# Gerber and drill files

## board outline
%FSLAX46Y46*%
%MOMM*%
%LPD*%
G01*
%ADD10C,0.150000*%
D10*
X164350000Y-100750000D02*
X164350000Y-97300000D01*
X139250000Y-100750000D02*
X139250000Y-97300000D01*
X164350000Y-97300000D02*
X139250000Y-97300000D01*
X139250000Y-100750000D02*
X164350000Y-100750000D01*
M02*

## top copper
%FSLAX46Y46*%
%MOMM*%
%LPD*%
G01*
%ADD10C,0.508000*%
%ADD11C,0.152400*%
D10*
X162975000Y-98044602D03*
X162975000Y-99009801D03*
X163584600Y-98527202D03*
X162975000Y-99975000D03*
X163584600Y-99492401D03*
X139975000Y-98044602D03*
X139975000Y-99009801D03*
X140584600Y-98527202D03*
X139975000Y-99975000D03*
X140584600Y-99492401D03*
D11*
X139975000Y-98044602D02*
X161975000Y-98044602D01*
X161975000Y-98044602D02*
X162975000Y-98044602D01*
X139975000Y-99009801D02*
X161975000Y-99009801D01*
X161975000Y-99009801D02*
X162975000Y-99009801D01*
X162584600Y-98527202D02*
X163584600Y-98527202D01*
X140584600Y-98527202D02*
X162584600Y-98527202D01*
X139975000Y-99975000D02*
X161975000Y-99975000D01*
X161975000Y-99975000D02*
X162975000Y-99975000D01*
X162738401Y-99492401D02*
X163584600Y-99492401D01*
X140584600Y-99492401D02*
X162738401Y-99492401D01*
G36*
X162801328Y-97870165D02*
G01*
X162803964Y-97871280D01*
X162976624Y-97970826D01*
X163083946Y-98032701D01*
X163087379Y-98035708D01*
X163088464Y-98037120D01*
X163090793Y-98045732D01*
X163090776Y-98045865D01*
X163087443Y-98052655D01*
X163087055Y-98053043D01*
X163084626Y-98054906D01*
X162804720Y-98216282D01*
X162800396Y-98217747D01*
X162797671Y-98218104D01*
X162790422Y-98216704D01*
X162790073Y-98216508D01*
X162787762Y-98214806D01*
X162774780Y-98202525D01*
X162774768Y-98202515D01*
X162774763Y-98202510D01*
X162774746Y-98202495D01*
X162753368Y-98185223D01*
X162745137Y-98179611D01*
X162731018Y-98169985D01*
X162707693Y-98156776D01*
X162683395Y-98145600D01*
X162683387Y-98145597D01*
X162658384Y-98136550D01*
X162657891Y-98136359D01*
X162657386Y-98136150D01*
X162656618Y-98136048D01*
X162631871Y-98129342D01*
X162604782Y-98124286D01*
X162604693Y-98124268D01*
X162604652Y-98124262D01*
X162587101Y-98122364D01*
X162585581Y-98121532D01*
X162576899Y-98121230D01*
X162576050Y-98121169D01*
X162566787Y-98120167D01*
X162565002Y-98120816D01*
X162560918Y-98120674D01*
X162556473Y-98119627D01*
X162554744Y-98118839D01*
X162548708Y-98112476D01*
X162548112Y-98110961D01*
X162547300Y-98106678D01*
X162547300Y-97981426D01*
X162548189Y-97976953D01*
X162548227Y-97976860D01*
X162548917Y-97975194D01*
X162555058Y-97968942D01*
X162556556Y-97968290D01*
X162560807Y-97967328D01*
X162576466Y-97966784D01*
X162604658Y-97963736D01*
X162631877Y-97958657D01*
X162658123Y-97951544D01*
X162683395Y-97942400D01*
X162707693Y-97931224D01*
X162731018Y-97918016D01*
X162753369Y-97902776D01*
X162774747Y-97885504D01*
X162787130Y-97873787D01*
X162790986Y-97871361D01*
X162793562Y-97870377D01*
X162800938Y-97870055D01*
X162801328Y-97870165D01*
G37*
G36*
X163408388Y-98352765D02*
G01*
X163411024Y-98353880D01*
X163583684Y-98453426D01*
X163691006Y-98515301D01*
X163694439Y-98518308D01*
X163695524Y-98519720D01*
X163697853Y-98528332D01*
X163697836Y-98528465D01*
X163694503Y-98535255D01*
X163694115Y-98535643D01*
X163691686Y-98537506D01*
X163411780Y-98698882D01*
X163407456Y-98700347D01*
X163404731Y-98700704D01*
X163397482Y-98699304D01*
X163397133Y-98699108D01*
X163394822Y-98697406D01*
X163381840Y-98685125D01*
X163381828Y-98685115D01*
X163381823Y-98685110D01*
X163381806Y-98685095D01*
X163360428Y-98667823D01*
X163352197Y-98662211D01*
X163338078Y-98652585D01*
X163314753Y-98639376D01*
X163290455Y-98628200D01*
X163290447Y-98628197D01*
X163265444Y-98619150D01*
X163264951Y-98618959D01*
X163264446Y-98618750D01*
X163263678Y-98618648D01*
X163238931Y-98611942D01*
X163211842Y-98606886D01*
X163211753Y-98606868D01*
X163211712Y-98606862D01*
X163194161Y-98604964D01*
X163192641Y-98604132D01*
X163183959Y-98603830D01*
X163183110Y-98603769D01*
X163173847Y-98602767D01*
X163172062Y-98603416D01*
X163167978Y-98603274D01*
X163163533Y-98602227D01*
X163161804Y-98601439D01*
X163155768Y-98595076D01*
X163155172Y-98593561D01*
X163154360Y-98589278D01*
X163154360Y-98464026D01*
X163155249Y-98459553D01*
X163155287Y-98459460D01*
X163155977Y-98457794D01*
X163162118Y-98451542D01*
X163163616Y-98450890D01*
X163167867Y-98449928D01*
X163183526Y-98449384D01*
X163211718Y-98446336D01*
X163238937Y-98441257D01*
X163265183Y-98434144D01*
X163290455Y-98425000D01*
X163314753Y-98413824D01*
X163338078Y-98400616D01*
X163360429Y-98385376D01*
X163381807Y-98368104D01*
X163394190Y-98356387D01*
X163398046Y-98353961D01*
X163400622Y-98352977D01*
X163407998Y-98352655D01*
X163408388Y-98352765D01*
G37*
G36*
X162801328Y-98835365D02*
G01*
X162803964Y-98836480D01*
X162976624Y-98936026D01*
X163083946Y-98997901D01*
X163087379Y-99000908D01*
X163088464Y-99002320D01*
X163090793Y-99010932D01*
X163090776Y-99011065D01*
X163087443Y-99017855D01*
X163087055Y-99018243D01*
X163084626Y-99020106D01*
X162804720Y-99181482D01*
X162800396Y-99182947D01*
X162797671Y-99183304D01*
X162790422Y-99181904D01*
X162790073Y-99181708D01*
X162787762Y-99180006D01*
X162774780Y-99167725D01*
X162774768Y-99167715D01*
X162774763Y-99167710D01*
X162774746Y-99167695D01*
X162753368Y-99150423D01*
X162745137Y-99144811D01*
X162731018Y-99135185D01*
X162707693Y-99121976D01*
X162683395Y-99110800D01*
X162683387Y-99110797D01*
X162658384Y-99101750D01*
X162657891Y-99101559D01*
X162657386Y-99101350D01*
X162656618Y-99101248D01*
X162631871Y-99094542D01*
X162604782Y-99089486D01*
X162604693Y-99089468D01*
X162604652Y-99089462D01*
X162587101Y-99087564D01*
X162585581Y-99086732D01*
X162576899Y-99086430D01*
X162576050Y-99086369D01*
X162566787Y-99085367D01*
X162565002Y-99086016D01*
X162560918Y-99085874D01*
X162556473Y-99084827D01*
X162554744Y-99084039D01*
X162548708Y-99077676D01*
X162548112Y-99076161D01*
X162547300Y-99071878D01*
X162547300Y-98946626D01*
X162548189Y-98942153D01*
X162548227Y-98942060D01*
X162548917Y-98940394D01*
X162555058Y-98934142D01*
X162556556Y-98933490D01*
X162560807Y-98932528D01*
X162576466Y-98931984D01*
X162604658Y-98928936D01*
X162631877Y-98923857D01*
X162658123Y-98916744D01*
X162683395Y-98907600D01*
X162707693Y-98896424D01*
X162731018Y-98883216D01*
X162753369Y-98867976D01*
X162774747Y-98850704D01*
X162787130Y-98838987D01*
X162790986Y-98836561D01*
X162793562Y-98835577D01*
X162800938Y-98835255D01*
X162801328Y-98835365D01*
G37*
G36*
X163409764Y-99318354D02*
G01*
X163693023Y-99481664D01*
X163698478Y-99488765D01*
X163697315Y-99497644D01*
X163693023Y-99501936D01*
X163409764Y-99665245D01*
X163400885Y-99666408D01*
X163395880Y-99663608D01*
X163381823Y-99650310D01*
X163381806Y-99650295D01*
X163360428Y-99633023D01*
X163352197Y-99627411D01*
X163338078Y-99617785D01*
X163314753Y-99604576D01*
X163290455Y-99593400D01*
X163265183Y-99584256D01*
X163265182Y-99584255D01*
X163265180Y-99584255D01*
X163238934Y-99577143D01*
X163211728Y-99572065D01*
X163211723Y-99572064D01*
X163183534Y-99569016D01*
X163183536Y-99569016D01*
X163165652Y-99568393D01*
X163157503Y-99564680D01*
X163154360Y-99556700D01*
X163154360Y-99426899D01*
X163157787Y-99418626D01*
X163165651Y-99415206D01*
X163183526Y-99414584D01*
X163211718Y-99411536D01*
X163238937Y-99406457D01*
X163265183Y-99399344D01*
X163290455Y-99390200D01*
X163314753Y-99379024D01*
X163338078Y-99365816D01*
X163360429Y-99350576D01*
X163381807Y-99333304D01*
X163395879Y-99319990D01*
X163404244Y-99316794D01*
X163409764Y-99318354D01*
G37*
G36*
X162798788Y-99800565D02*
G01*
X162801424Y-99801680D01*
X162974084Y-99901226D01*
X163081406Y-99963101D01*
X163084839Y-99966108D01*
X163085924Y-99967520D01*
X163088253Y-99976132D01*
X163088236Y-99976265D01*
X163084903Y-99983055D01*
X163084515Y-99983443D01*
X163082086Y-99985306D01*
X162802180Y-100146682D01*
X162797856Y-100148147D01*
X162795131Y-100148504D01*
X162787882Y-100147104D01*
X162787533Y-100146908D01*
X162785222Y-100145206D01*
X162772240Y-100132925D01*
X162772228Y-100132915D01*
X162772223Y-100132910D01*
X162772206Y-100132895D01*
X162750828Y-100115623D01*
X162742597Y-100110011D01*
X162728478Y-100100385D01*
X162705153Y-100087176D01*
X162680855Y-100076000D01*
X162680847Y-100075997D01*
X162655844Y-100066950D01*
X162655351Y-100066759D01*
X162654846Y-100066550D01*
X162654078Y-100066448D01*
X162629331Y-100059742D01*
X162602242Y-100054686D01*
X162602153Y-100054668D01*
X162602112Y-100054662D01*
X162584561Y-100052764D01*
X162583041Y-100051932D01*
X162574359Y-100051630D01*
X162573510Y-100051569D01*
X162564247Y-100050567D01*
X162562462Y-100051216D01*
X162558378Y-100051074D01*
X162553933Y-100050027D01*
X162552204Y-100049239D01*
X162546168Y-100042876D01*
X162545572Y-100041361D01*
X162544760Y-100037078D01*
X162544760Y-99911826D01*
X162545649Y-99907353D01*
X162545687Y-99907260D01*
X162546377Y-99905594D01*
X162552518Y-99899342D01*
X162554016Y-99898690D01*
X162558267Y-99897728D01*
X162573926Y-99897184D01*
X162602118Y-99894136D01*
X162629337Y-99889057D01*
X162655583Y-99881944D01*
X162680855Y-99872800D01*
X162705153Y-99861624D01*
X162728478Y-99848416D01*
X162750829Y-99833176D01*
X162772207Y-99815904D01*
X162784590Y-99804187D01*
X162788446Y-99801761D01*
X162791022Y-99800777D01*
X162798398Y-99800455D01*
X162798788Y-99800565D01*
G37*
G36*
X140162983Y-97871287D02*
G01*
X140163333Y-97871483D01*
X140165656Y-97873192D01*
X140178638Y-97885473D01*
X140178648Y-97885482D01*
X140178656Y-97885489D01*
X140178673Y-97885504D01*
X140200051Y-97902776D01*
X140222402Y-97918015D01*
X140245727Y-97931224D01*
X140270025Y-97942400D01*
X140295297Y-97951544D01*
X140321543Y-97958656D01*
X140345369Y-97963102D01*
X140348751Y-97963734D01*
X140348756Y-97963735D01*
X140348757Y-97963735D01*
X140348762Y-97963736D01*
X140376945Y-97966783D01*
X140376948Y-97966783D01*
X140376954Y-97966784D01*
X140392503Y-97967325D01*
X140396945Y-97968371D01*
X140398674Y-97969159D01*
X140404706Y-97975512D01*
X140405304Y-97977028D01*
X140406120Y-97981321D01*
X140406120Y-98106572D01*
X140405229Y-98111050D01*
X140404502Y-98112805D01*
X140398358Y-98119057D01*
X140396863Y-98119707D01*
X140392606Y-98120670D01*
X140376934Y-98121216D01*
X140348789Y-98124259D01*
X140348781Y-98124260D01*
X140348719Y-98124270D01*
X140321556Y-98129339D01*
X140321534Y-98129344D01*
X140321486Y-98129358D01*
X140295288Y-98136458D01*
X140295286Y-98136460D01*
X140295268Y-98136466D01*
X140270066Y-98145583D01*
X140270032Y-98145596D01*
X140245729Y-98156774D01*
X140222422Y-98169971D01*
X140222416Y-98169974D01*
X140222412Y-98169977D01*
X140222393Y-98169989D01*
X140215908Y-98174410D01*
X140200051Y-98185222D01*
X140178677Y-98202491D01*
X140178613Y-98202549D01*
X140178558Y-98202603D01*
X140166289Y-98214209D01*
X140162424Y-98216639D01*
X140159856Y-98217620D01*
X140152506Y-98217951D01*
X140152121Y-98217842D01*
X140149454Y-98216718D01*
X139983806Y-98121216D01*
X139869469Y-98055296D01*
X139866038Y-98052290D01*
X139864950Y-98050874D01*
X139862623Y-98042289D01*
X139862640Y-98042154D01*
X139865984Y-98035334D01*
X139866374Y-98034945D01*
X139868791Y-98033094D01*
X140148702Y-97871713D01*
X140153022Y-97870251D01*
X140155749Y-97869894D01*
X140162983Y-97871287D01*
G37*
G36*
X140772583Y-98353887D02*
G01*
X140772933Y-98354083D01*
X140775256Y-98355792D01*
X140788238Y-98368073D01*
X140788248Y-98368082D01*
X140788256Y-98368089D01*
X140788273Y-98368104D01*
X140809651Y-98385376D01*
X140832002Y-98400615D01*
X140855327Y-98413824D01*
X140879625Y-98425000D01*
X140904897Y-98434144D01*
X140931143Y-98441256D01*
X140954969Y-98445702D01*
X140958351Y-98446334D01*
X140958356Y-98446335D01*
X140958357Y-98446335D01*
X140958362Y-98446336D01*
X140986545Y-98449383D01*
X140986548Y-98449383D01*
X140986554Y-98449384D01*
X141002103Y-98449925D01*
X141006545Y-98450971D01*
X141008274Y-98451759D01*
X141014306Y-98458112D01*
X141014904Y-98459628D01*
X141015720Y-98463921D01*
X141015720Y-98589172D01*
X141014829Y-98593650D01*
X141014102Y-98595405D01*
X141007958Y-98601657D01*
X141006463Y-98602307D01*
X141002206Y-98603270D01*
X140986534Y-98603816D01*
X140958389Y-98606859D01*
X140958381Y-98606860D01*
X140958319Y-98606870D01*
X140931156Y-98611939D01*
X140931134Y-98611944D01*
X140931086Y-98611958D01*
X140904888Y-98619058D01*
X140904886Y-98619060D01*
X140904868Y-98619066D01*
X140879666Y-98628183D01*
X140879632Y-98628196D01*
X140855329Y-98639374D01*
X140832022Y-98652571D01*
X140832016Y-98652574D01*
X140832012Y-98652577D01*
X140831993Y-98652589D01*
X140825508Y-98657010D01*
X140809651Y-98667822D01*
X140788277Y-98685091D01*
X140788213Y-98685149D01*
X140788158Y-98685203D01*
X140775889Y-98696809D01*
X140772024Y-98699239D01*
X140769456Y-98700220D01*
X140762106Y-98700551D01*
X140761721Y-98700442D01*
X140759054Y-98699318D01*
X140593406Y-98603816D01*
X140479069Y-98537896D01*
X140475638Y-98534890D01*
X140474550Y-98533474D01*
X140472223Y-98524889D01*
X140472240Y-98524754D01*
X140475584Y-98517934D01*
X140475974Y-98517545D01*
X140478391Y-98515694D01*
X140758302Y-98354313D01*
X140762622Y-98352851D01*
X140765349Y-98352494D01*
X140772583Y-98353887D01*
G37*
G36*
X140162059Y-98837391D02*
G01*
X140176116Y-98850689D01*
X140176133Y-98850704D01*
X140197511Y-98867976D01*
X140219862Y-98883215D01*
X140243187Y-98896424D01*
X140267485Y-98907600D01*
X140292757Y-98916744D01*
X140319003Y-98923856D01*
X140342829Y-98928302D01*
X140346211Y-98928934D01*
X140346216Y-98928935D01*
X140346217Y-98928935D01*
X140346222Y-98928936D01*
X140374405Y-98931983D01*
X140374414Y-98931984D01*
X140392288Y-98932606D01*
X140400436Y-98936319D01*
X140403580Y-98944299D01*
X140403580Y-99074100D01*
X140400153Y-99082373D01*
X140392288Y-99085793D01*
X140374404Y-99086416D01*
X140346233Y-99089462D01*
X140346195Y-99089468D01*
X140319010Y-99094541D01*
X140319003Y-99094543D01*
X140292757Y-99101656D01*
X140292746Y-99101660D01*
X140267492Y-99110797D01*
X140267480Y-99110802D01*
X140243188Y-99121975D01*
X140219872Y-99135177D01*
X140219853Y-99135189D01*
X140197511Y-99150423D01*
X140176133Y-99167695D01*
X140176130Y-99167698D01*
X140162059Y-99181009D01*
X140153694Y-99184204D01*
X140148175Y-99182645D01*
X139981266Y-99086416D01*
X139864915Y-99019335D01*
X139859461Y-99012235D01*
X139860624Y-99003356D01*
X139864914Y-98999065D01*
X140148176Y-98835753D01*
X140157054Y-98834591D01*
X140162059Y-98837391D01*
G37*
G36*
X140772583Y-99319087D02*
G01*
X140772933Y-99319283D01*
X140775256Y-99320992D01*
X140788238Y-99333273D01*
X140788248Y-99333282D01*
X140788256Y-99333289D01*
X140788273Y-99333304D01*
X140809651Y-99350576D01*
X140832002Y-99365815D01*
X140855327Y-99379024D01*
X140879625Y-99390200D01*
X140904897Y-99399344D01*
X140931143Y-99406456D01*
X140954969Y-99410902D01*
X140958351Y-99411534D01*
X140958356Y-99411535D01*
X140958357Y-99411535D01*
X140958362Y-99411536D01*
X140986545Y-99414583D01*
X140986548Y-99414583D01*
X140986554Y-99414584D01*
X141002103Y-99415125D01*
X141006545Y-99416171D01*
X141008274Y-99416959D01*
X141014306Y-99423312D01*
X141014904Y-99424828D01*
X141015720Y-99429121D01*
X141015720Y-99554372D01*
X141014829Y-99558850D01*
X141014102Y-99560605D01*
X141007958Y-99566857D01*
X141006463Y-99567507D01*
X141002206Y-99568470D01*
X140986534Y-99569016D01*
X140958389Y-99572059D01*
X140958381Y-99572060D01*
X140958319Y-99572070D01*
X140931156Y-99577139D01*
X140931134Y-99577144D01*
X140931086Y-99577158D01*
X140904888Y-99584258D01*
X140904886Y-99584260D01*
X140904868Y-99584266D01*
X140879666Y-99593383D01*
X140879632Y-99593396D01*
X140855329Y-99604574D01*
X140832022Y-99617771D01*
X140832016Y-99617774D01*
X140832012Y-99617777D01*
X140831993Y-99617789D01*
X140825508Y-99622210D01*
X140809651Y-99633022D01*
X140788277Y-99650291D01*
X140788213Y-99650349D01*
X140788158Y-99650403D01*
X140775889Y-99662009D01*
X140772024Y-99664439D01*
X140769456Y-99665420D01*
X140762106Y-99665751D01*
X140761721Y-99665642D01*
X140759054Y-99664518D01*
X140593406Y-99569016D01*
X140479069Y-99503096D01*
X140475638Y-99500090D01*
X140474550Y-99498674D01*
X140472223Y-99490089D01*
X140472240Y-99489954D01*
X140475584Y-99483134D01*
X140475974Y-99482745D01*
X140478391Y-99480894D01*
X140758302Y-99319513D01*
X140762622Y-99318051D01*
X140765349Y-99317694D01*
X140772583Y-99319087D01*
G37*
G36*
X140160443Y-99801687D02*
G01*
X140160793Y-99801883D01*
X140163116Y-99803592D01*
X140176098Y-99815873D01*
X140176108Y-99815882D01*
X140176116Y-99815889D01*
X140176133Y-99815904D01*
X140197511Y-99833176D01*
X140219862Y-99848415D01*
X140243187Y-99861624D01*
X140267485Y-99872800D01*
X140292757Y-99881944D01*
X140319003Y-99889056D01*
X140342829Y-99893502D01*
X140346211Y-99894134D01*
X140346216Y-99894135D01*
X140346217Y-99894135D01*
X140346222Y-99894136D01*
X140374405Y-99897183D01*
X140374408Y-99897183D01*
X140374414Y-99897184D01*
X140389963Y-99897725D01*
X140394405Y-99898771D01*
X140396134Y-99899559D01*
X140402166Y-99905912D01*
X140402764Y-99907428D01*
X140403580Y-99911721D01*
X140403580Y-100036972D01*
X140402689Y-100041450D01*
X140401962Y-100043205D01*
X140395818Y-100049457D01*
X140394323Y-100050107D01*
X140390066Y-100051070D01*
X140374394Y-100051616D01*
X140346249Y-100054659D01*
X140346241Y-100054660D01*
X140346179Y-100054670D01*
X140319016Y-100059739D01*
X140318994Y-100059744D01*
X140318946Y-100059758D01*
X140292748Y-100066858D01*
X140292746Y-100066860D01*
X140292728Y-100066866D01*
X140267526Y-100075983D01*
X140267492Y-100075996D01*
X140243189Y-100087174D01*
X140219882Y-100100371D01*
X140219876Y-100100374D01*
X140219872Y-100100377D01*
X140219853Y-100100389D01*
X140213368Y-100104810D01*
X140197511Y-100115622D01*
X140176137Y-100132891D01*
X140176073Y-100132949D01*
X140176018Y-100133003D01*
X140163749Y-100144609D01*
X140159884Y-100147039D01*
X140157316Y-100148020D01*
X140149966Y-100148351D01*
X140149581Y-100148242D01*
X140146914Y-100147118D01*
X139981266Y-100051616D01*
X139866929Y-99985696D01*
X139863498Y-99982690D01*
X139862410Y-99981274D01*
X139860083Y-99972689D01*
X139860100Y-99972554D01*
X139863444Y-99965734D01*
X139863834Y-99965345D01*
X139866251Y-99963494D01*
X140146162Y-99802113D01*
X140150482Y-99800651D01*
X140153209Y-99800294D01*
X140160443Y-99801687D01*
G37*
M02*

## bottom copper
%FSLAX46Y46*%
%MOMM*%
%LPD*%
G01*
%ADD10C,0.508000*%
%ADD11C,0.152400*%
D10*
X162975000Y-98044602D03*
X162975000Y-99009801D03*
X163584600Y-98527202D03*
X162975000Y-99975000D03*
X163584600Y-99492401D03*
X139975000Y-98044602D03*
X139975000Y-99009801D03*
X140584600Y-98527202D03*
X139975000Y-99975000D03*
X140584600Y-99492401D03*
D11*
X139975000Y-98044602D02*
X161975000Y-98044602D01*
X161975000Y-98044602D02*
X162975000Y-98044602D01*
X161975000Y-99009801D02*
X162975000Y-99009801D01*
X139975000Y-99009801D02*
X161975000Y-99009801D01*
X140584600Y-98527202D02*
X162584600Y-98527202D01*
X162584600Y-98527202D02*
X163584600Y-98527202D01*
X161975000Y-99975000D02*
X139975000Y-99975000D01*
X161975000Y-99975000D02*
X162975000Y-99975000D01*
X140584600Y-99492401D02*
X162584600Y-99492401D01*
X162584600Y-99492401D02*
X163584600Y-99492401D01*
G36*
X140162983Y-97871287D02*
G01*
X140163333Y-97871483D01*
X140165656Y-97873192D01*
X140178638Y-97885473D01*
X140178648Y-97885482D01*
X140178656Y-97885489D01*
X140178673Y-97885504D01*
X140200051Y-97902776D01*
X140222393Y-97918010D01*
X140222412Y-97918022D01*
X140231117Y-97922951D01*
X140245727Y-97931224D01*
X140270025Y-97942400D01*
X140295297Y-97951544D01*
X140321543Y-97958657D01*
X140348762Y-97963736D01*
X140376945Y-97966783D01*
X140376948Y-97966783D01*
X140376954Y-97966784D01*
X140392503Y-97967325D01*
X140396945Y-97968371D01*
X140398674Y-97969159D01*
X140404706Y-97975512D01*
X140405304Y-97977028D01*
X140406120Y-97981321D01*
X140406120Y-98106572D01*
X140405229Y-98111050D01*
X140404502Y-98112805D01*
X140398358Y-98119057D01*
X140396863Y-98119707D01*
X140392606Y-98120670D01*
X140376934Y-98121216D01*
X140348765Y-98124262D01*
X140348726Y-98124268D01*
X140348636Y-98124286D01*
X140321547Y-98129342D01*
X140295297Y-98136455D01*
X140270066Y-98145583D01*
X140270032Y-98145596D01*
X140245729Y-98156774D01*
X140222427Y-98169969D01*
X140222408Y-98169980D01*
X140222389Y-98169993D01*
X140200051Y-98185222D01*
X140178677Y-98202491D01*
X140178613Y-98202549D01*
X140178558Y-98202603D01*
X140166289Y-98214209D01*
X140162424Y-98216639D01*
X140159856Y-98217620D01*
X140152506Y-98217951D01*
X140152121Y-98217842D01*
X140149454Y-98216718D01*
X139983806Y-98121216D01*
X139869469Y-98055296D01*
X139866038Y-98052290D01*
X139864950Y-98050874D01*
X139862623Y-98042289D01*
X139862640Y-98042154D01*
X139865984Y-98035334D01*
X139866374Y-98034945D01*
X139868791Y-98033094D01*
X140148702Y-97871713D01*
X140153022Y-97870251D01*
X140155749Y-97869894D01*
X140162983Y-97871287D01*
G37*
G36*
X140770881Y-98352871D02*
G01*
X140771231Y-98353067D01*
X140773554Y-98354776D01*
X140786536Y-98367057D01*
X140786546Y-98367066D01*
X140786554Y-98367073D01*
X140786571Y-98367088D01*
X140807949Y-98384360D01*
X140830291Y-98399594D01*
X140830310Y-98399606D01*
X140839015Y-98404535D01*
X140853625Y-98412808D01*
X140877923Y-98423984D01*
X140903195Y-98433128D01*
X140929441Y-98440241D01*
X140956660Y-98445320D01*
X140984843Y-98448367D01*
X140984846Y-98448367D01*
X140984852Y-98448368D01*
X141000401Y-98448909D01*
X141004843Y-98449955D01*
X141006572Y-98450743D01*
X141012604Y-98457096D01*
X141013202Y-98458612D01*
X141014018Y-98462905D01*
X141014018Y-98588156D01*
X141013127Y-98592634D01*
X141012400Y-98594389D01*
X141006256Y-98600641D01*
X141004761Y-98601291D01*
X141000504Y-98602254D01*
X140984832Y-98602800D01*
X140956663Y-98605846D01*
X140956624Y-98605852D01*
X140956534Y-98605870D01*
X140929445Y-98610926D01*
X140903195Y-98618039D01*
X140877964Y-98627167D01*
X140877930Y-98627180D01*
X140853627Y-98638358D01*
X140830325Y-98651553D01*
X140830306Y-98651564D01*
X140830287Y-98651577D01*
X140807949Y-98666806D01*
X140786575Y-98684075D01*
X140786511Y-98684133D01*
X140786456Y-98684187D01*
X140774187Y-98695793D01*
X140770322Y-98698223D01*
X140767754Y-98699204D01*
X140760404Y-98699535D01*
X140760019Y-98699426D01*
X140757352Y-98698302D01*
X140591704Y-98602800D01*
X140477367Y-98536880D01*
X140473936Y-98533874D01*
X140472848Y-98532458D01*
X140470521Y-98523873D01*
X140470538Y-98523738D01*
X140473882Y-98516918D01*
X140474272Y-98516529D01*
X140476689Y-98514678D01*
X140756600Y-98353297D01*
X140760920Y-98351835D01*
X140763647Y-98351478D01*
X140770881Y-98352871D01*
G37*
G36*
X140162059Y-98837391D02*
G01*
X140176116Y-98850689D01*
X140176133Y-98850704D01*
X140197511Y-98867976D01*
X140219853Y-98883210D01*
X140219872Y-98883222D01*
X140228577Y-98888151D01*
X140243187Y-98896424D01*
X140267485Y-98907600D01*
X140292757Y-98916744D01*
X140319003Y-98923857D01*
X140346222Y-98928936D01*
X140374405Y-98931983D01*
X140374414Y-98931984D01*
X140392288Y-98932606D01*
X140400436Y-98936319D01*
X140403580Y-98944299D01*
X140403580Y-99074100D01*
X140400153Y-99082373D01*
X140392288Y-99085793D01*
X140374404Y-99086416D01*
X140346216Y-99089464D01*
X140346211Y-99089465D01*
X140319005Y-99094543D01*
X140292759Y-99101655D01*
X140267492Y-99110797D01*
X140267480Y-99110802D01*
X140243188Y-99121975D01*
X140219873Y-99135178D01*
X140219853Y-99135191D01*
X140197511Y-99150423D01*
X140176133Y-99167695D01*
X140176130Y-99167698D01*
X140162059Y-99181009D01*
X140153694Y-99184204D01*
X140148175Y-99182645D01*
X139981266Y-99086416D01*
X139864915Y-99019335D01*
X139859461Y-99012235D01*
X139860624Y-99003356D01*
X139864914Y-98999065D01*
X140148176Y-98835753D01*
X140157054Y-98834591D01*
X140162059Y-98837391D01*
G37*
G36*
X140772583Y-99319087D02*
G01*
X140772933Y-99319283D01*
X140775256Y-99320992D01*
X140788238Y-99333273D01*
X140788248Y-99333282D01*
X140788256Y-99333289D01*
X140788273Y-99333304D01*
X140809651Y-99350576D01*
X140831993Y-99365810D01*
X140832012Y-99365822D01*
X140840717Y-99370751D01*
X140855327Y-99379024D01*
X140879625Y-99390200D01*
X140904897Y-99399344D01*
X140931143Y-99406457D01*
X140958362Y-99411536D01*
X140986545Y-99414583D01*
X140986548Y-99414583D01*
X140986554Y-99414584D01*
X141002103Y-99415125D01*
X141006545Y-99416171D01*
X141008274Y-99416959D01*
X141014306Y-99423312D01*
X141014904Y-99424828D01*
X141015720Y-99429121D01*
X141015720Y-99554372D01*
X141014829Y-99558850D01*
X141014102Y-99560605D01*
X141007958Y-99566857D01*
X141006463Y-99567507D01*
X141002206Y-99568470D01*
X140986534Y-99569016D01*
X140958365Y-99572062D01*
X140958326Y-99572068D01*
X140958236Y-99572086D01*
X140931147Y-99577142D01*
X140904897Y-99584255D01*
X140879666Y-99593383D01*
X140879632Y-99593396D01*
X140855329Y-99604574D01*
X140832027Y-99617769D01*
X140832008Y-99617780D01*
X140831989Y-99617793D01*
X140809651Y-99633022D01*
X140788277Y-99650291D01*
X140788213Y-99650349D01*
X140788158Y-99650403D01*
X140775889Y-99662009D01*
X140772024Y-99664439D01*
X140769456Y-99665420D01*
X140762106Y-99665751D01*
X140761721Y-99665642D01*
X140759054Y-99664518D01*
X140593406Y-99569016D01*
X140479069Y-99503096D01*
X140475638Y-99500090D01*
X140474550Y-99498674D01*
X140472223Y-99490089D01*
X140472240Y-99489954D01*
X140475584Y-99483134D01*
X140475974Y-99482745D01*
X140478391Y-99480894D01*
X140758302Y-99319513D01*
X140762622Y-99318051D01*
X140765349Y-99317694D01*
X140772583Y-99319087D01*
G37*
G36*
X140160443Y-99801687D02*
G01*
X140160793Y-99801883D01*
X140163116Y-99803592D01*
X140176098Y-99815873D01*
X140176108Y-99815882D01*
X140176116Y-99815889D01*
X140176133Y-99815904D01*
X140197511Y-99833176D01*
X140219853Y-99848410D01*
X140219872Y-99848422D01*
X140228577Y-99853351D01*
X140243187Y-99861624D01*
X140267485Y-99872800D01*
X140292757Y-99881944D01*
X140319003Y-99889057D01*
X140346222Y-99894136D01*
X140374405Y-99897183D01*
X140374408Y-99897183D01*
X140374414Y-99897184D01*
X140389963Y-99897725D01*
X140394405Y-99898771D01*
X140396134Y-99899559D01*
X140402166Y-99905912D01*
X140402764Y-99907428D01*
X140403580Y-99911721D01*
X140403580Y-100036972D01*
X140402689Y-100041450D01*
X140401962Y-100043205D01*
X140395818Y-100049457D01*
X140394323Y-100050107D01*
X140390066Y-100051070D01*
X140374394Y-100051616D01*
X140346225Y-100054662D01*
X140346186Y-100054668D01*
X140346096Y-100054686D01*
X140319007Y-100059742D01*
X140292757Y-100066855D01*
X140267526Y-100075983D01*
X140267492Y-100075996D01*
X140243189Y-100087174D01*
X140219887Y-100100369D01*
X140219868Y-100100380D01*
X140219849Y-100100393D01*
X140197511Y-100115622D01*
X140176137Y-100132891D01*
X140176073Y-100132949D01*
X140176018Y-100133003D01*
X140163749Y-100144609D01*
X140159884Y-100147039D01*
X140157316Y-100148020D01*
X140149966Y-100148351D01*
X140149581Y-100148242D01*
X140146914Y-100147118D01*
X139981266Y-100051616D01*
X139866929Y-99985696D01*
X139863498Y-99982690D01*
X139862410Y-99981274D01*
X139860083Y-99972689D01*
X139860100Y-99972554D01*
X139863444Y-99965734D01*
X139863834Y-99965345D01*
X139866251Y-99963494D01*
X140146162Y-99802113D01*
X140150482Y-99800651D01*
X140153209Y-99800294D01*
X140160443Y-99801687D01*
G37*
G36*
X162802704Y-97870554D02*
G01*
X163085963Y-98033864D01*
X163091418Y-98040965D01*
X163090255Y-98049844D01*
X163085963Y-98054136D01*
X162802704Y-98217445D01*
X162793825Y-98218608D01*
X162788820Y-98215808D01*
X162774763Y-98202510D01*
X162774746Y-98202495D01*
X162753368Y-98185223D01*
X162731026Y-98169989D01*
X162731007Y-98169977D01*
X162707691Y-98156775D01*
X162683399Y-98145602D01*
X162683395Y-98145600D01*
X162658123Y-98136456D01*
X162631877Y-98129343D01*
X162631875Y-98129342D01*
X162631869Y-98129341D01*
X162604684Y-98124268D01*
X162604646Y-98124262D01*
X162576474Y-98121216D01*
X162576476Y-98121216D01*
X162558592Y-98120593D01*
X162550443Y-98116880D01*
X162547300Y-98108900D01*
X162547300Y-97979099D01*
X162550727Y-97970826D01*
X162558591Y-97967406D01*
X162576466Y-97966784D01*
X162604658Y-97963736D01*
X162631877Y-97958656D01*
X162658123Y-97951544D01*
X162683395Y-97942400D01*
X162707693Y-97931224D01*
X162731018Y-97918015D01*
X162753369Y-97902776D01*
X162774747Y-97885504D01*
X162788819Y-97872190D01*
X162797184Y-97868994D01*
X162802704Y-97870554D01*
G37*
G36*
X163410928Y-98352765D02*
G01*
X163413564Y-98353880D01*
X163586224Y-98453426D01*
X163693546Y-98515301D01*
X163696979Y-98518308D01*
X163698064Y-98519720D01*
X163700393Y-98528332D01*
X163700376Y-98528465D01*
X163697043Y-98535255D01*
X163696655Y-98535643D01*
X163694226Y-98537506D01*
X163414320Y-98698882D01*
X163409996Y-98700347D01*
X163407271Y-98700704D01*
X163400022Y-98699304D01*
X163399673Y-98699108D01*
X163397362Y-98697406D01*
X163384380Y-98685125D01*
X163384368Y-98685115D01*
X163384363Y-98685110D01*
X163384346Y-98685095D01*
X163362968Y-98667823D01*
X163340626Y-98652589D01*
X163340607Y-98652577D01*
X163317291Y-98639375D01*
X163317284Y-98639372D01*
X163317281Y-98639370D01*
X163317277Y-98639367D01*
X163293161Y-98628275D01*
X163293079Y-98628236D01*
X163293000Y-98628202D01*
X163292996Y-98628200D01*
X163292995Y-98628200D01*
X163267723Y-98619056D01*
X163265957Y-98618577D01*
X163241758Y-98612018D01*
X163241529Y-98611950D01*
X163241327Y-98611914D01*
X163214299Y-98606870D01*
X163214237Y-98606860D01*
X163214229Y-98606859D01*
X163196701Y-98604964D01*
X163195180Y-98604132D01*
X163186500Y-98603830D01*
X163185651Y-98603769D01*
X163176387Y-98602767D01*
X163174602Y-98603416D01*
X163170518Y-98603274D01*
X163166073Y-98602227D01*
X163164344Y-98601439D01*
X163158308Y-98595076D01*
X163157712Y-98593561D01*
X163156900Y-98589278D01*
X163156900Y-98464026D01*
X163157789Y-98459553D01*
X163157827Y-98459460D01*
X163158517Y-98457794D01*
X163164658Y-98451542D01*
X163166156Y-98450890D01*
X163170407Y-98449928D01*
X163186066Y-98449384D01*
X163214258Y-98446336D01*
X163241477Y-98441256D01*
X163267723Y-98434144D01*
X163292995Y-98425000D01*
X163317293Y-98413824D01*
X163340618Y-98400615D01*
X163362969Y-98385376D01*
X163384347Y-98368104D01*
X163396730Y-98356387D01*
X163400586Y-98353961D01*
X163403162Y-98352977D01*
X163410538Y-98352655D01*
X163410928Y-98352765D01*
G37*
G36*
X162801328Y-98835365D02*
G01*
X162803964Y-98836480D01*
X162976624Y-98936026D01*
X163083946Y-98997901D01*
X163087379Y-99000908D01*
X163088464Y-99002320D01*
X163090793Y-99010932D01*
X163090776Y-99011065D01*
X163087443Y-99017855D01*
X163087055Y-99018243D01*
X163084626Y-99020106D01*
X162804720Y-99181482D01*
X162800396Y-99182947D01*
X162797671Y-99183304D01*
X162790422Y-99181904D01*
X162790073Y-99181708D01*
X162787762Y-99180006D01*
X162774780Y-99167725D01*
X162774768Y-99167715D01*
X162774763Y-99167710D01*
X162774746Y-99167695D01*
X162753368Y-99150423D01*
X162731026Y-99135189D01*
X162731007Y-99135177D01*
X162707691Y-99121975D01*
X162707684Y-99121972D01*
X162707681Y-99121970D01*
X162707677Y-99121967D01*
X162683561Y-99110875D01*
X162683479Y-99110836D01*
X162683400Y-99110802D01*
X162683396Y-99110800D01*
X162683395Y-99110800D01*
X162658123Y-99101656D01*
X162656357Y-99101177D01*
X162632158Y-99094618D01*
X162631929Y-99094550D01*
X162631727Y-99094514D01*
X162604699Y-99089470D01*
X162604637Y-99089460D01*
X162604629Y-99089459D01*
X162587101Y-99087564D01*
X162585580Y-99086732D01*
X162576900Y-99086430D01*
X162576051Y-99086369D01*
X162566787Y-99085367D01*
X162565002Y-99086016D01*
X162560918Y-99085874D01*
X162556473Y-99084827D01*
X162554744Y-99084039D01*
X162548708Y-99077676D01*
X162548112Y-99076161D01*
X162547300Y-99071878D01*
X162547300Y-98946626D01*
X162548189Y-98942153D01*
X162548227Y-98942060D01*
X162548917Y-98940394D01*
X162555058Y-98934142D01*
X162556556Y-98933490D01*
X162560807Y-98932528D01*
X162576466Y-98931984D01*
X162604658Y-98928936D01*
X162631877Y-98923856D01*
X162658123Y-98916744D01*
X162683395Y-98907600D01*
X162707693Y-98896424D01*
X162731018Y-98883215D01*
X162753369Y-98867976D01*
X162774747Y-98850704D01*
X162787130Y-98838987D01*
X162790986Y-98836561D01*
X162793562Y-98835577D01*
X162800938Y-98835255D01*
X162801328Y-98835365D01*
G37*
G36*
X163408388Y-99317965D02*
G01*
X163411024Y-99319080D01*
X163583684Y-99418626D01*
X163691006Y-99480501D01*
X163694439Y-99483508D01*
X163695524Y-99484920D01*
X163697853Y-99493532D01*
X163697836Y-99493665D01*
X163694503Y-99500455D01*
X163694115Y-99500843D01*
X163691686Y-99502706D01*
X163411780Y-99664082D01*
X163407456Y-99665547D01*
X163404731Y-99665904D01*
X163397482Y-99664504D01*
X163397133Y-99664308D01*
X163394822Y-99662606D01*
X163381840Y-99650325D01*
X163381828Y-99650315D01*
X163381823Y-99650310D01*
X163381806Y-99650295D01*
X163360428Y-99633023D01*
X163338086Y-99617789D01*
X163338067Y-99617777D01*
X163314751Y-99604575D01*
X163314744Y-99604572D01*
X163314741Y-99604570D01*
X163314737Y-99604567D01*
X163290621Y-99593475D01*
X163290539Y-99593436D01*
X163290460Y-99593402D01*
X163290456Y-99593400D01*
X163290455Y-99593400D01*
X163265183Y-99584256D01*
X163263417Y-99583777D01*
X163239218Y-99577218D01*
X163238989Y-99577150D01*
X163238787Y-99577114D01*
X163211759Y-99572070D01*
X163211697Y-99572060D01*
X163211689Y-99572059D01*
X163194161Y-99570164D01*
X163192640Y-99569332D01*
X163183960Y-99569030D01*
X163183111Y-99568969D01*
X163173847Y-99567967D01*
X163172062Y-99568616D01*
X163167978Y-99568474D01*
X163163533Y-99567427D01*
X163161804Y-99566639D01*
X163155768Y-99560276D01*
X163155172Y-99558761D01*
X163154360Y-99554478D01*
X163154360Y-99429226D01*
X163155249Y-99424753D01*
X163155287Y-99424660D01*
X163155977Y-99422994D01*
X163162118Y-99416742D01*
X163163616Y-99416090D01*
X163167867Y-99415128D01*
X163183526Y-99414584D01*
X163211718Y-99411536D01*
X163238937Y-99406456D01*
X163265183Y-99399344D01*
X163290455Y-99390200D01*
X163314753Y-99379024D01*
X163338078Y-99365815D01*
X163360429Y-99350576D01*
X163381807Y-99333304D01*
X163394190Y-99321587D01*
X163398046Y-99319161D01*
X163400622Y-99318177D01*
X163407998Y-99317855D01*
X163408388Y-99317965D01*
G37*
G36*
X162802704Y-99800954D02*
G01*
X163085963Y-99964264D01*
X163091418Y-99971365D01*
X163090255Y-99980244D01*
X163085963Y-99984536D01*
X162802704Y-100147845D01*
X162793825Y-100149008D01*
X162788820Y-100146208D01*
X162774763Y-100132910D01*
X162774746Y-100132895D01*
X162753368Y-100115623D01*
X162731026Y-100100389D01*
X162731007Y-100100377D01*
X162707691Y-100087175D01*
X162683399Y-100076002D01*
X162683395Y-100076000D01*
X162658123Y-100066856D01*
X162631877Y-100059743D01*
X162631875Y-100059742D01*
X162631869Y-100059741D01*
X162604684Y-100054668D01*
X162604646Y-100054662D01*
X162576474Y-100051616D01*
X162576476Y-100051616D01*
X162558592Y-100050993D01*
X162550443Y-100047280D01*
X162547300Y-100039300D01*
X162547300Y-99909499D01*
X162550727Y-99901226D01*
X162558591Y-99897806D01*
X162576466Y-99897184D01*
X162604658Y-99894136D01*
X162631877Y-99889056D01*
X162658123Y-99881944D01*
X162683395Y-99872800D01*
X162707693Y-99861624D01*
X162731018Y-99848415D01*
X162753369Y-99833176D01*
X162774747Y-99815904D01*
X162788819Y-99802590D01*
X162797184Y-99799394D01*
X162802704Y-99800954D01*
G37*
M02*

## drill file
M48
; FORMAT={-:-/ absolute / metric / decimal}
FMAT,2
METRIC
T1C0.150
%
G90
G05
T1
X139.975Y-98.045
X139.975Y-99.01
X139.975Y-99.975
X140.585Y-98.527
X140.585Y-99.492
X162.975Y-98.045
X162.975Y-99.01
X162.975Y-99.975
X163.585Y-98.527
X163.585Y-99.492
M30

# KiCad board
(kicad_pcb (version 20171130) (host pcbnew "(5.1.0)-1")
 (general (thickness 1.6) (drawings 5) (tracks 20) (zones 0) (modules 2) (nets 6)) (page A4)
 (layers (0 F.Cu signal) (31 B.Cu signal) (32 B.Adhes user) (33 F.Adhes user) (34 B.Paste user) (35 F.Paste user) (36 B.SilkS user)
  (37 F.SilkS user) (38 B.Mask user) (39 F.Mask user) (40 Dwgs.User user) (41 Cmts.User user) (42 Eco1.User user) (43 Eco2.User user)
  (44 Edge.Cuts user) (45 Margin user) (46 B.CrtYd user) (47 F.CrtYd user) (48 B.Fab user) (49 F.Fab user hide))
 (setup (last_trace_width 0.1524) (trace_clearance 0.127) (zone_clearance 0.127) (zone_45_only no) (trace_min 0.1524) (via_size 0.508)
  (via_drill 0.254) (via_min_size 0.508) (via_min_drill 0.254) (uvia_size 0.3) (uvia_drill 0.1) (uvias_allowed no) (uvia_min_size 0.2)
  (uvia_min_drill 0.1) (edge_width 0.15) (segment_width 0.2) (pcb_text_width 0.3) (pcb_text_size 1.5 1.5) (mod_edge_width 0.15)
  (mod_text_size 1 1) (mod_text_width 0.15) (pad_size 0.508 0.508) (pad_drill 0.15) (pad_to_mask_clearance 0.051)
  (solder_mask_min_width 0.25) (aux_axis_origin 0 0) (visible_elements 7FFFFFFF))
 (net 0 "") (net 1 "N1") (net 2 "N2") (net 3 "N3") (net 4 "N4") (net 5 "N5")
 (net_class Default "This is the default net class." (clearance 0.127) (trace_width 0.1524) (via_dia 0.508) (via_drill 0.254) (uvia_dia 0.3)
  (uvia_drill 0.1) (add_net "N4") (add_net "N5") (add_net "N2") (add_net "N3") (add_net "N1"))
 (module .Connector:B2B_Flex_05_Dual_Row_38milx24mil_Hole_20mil (layer F.Cu) (at 163 100 90)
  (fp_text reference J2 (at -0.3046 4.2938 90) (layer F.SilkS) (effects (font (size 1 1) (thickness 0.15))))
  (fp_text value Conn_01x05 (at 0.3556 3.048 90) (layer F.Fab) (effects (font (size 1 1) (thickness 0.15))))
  (pad 5 thru_hole circle (at 1.955398 -0.025 90) (size 0.508 0.508) (drill 0.15) (layers *.Cu *.Mask) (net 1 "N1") (zone_connect 2))
  (pad 3 thru_hole circle (at 0.990199 -0.025 90) (size 0.508 0.508) (drill 0.15) (layers *.Cu *.Mask) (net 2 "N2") (zone_connect 2))
  (pad 4 thru_hole circle (at 1.472798 0.5846 90) (size 0.508 0.508) (drill 0.15) (layers *.Cu *.Mask) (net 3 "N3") (zone_connect 2))
  (pad 1 thru_hole circle (at 0.025 -0.025 90) (size 0.508 0.508) (drill 0.15) (layers *.Cu *.Mask) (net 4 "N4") (zone_connect 2))
  (pad 2 thru_hole circle (at 0.507599 0.5846 90) (size 0.508 0.508) (drill 0.15) (layers *.Cu *.Mask) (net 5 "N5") (zone_connect 2)))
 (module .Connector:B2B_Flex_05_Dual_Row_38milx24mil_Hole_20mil (layer F.Cu) (at 140 100 90)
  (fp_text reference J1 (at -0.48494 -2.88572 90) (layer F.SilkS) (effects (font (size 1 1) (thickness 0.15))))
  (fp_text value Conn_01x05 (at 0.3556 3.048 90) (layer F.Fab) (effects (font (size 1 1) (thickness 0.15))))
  (pad 5 thru_hole circle (at 1.955398 -0.025 90) (size 0.508 0.508) (drill 0.15) (layers *.Cu *.Mask) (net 1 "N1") (zone_connect 2))
  (pad 3 thru_hole circle (at 0.990199 -0.025 90) (size 0.508 0.508) (drill 0.15) (layers *.Cu *.Mask) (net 2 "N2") (zone_connect 2))
  (pad 4 thru_hole circle (at 1.472798 0.5846 90) (size 0.508 0.508) (drill 0.15) (layers *.Cu *.Mask) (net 3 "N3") (zone_connect 2))
  (pad 1 thru_hole circle (at 0.025 -0.025 90) (size 0.508 0.508) (drill 0.15) (layers *.Cu *.Mask) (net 4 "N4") (zone_connect 2))
  (pad 2 thru_hole circle (at 0.507599 0.5846 90) (size 0.508 0.508) (drill 0.15) (layers *.Cu *.Mask) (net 5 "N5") (zone_connect 2)))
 (gr_line (start 164.35 100.75) (end 164.35 97.3) (layer Edge.Cuts) (width 0.15))
 (gr_line (start 139.25 100.75) (end 139.25 97.3) (layer Edge.Cuts) (width 0.15))
 (gr_line (start 164.35 97.3) (end 139.25 97.3) (layer Edge.Cuts) (width 0.15))
 (gr_line (start 139.25 100.75) (end 164.35 100.75) (layer Edge.Cuts) (width 0.15))
 (segment (start 139.975 98.044602) (end 161.975 98.044602) (width 0.1524) (layer F.Cu) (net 1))
 (segment (start 139.975 98.044602) (end 161.975 98.044602) (width 0.1524) (layer B.Cu) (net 1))
 (segment (start 161.975 98.044602) (end 162.975 98.044602) (width 0.1524) (layer B.Cu) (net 1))
 (segment (start 161.975 98.044602) (end 162.975 98.044602) (width 0.1524) (layer F.Cu) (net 1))
 (segment (start 139.975 99.009801) (end 161.975 99.009801) (width 0.1524) (layer F.Cu) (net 2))
 (segment (start 161.975 99.009801) (end 162.975 99.009801) (width 0.1524) (layer B.Cu) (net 2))
 (segment (start 139.975 99.009801) (end 161.975 99.009801) (width 0.1524) (layer B.Cu) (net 2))
 (segment (start 161.975 99.009801) (end 162.975 99.009801) (width 0.1524) (layer F.Cu) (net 2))
 (segment (start 140.5846 98.527202) (end 162.5846 98.527202) (width 0.1524) (layer B.Cu) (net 3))
 (segment (start 162.5846 98.527202) (end 163.5846 98.527202) (width 0.1524) (layer B.Cu) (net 3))
 (segment (start 162.5846 98.527202) (end 163.5846 98.527202) (width 0.1524) (layer F.Cu) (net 3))
 (segment (start 140.5846 98.527202) (end 162.5846 98.527202) (width 0.1524) (layer F.Cu) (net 3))
 (segment (start 139.975 99.975) (end 161.975 99.975) (width 0.1524) (layer F.Cu) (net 4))
 (segment (start 161.975 99.975) (end 139.975 99.975) (width 0.1524) (layer B.Cu) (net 4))
 (segment (start 161.975 99.975) (end 162.975 99.975) (width 0.1524) (layer B.Cu) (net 4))
 (segment (start 161.975 99.975) (end 162.975 99.975) (width 0.1524) (layer F.Cu) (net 4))
 (segment (start 140.5846 99.492401) (end 162.5846 99.492401) (width 0.1524) (layer B.Cu) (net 5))
 (segment (start 162.5846 99.492401) (end 163.5846 99.492401) (width 0.1524) (layer B.Cu) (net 5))
 (segment (start 162.738401 99.492401) (end 163.5846 99.492401) (width 0.1524) (layer F.Cu) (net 5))
 (segment (start 140.5846 99.492401) (end 162.738401 99.492401) (width 0.1524) (layer F.Cu) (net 5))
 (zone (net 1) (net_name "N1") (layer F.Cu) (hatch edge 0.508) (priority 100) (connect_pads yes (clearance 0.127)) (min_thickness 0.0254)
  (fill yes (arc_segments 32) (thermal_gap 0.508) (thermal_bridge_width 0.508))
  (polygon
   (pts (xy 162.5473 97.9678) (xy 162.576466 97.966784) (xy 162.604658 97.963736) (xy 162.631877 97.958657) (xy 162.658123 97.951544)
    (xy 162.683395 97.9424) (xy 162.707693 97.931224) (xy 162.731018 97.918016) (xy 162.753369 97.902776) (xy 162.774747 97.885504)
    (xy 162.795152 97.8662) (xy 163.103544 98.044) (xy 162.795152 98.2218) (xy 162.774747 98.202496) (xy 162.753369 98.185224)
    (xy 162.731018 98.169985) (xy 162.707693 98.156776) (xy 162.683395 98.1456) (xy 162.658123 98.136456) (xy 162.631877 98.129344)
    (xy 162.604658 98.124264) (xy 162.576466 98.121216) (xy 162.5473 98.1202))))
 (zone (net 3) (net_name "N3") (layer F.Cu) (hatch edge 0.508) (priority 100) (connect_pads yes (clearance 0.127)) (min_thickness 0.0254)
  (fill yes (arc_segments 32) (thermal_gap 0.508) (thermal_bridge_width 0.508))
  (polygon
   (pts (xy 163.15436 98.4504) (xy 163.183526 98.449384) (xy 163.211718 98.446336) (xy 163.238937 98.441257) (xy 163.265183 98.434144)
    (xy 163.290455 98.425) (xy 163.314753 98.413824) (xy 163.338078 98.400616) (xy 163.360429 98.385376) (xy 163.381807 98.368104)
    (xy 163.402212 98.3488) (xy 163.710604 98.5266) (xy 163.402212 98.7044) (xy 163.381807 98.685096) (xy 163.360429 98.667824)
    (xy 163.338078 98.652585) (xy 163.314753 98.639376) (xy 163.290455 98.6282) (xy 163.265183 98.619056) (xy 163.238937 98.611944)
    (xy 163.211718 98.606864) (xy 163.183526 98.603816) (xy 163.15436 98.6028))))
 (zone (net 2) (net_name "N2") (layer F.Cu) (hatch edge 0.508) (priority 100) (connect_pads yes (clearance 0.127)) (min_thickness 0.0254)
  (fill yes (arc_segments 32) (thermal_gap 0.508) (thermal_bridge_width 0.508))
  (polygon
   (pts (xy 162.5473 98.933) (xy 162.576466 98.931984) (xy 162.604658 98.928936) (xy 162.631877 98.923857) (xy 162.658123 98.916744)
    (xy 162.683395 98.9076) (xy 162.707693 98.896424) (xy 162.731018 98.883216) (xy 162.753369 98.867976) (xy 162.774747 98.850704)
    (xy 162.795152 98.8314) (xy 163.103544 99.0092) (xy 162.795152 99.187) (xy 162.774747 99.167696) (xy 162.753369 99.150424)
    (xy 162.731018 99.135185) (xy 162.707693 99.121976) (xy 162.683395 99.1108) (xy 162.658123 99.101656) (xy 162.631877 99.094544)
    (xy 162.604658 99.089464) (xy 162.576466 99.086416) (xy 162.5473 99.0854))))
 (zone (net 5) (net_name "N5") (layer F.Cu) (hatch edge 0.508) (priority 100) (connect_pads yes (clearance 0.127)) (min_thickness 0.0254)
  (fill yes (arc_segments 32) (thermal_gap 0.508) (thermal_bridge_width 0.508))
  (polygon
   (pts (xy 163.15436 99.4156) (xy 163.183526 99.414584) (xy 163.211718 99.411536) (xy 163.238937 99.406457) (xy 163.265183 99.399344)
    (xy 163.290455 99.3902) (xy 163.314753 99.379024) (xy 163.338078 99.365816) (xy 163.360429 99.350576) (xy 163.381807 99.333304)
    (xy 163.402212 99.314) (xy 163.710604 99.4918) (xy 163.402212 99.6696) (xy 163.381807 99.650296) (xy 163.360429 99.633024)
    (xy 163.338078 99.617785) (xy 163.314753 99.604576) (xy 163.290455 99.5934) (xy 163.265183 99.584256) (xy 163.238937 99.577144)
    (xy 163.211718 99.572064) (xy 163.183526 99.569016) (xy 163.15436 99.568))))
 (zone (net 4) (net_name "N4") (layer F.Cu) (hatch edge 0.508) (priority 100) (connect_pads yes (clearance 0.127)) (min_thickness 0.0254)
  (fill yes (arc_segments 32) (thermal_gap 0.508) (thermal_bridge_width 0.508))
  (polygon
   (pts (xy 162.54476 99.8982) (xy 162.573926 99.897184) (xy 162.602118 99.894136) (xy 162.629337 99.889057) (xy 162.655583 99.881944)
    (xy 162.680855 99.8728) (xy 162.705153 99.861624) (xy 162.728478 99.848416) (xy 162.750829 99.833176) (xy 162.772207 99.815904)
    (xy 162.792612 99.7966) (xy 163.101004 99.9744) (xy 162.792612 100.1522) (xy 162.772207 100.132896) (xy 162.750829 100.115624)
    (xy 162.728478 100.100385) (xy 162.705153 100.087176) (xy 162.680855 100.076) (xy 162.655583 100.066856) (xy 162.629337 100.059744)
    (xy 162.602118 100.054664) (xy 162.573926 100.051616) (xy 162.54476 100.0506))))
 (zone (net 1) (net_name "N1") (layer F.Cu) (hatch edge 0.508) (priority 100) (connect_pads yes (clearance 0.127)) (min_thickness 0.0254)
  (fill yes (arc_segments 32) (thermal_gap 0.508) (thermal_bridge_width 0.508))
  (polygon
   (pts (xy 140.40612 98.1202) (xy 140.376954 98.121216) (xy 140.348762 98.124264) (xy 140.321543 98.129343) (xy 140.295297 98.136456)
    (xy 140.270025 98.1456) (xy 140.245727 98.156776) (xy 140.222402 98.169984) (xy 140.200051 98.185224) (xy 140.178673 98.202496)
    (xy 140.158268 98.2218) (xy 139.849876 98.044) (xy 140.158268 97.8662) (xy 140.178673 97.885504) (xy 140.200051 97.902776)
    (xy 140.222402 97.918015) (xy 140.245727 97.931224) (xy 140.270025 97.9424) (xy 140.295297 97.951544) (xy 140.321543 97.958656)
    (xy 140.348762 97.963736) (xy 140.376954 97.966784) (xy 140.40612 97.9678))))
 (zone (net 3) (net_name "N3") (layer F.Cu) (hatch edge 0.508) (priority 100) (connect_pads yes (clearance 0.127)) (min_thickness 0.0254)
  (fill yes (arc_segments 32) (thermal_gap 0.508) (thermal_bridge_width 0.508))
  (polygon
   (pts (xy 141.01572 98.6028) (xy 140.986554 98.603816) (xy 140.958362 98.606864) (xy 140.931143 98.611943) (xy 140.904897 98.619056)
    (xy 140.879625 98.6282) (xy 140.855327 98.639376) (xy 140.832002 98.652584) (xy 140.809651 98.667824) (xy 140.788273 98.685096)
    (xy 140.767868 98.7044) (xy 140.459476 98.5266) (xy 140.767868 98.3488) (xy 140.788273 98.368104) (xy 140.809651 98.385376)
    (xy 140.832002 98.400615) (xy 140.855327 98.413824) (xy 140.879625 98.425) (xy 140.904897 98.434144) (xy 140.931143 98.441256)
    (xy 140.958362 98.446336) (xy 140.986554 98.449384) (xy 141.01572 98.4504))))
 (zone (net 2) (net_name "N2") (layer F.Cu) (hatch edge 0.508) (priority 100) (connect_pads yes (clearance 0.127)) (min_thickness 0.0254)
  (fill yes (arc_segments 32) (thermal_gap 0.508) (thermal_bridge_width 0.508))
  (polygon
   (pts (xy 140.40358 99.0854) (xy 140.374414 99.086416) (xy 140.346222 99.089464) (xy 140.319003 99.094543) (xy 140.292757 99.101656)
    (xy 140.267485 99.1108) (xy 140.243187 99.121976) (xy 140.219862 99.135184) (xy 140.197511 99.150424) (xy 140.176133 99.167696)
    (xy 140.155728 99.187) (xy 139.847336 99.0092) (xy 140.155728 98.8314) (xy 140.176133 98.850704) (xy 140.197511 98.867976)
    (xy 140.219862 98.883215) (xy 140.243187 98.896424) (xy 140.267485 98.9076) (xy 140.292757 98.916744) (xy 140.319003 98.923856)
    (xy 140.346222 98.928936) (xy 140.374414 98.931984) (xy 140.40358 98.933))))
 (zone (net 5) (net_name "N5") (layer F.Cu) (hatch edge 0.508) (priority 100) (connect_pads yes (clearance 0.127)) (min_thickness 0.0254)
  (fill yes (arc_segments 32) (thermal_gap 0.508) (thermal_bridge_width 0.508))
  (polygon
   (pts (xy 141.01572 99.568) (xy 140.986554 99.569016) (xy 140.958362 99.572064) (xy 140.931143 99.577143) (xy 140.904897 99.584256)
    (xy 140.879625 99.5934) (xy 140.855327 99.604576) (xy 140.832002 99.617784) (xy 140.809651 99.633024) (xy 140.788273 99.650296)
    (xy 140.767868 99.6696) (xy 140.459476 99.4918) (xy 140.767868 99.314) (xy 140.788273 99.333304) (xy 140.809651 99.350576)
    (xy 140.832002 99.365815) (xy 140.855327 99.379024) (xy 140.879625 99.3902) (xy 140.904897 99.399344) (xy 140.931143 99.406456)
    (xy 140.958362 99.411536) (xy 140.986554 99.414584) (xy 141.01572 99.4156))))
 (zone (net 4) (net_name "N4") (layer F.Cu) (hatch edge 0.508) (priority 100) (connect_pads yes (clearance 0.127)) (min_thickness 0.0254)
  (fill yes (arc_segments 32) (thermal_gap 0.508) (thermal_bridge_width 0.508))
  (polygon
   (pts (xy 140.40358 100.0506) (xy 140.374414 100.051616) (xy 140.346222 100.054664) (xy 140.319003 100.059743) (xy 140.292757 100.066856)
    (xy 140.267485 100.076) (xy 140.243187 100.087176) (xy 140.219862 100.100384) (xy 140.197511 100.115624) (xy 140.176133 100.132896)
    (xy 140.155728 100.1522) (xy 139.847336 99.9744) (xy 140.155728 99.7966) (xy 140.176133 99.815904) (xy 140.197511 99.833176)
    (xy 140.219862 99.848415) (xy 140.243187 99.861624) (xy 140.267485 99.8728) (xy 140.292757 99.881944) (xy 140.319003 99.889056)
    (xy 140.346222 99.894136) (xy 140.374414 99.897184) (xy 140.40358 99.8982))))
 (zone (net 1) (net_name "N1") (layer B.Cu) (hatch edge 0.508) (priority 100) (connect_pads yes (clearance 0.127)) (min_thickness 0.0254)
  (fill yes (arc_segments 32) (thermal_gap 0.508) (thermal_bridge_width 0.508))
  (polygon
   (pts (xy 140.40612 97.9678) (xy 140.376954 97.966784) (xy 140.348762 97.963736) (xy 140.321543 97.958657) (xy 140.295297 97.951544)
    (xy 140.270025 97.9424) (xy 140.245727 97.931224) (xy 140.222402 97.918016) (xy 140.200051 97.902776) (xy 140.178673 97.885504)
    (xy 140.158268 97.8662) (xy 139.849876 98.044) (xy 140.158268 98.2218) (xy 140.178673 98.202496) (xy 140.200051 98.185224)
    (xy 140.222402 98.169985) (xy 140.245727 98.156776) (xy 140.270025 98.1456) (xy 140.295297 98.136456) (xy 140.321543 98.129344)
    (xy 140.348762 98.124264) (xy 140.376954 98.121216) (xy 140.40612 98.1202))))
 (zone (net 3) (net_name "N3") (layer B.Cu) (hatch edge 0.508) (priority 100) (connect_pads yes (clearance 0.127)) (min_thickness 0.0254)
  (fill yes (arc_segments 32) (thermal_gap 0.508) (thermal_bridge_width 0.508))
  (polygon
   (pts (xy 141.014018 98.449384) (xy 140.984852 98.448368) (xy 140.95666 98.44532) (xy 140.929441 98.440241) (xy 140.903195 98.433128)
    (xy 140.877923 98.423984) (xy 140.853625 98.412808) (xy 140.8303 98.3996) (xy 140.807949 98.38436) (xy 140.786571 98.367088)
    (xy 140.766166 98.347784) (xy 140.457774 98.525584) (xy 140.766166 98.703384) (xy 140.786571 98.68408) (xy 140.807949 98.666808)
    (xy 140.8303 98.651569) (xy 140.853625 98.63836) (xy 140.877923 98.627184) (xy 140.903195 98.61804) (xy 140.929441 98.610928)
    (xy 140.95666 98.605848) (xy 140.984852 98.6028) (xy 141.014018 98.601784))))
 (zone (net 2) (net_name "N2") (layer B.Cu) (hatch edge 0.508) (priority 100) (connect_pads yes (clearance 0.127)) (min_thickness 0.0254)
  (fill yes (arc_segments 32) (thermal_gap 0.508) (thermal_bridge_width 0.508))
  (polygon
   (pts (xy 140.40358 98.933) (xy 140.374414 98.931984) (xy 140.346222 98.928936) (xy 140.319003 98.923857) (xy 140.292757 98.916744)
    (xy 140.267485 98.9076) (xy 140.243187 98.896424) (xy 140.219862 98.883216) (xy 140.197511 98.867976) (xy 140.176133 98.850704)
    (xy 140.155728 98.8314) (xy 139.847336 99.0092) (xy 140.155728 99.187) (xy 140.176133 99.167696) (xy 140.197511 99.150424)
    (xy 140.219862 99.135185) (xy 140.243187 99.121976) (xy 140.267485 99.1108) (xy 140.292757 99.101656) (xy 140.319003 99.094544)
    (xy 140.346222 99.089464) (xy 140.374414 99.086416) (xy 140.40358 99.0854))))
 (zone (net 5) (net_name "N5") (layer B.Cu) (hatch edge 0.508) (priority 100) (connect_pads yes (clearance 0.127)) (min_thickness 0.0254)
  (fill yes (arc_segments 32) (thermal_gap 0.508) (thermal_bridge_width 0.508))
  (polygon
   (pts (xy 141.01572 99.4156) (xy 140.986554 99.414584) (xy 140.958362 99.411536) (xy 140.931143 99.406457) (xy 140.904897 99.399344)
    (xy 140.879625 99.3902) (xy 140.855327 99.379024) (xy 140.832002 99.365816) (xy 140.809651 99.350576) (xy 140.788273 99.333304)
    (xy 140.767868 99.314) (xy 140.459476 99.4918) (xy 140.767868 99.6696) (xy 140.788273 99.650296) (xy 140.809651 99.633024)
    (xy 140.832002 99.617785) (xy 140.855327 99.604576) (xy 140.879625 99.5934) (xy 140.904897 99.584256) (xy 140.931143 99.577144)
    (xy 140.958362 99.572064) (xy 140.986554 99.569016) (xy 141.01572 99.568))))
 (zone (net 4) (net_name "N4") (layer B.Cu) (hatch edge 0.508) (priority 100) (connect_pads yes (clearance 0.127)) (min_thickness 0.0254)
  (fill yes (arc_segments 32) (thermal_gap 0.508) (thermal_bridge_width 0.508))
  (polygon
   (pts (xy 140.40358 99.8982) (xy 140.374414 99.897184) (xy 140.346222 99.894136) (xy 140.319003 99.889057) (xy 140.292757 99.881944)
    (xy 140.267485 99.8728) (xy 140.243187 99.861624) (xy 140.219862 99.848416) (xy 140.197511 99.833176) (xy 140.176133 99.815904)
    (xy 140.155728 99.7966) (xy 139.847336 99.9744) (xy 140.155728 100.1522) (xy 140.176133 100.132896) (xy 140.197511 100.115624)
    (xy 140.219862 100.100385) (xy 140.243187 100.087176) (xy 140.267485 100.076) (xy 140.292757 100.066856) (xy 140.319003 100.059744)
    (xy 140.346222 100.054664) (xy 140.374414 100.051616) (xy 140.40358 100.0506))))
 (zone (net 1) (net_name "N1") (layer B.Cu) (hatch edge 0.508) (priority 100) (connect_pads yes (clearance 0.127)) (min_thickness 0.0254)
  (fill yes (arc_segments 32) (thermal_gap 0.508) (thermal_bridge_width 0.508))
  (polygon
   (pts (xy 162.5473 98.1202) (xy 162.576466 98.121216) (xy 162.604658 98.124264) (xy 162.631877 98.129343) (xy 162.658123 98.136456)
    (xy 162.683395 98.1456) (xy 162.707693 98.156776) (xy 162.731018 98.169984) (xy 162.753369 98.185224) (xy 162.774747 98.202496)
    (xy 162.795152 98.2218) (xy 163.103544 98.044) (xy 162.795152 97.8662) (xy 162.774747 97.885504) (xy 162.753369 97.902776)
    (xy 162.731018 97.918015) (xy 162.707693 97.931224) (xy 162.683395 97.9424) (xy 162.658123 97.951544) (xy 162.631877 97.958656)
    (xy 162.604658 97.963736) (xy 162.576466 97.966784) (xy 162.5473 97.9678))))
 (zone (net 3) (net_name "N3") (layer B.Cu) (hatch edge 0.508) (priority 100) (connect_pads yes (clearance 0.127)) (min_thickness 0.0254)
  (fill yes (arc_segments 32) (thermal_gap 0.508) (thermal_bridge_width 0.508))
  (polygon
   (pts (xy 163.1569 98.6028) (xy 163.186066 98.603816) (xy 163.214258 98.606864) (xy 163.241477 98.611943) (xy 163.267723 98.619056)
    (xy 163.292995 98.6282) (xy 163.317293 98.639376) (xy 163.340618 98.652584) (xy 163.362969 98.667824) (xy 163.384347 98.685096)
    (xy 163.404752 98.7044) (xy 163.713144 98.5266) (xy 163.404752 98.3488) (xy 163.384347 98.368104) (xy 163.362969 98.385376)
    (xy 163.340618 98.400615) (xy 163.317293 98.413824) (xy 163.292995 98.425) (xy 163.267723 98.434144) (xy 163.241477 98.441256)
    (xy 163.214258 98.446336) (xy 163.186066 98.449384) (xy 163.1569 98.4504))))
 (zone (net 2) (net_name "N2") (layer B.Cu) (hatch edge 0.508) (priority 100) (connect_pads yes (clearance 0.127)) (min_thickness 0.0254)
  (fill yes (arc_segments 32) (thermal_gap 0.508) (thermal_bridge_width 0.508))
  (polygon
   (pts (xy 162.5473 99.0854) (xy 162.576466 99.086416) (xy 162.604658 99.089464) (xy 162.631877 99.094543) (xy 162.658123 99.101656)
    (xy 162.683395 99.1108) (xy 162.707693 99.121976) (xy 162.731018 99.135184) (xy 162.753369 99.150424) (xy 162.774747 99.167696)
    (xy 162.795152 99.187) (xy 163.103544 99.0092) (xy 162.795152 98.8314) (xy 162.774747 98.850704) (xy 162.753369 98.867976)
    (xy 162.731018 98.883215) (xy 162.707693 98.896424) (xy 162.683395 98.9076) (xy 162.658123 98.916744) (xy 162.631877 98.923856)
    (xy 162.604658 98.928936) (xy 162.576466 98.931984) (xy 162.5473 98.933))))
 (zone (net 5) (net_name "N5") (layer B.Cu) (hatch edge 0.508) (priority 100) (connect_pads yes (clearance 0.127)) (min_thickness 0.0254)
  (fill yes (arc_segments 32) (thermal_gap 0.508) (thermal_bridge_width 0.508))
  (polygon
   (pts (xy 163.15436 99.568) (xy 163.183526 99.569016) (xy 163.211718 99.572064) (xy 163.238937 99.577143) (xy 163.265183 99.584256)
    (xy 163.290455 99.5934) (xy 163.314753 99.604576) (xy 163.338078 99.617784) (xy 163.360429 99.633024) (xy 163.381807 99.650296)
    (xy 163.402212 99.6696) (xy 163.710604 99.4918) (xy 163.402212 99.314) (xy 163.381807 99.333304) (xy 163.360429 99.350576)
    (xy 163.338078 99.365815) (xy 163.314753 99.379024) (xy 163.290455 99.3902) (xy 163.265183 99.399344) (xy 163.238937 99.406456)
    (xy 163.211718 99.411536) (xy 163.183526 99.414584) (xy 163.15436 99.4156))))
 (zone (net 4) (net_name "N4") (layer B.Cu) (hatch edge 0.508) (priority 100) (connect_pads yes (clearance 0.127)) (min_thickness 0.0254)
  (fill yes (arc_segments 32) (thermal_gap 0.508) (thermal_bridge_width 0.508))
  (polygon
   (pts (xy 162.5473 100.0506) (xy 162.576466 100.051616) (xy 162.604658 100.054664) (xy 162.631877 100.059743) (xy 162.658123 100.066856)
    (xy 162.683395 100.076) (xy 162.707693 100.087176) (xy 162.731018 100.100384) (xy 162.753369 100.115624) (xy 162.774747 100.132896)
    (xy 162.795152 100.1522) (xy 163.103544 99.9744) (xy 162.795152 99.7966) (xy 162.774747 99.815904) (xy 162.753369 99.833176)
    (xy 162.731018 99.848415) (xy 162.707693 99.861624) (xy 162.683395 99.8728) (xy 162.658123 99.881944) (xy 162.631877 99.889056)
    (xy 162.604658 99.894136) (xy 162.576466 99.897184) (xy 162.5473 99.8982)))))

